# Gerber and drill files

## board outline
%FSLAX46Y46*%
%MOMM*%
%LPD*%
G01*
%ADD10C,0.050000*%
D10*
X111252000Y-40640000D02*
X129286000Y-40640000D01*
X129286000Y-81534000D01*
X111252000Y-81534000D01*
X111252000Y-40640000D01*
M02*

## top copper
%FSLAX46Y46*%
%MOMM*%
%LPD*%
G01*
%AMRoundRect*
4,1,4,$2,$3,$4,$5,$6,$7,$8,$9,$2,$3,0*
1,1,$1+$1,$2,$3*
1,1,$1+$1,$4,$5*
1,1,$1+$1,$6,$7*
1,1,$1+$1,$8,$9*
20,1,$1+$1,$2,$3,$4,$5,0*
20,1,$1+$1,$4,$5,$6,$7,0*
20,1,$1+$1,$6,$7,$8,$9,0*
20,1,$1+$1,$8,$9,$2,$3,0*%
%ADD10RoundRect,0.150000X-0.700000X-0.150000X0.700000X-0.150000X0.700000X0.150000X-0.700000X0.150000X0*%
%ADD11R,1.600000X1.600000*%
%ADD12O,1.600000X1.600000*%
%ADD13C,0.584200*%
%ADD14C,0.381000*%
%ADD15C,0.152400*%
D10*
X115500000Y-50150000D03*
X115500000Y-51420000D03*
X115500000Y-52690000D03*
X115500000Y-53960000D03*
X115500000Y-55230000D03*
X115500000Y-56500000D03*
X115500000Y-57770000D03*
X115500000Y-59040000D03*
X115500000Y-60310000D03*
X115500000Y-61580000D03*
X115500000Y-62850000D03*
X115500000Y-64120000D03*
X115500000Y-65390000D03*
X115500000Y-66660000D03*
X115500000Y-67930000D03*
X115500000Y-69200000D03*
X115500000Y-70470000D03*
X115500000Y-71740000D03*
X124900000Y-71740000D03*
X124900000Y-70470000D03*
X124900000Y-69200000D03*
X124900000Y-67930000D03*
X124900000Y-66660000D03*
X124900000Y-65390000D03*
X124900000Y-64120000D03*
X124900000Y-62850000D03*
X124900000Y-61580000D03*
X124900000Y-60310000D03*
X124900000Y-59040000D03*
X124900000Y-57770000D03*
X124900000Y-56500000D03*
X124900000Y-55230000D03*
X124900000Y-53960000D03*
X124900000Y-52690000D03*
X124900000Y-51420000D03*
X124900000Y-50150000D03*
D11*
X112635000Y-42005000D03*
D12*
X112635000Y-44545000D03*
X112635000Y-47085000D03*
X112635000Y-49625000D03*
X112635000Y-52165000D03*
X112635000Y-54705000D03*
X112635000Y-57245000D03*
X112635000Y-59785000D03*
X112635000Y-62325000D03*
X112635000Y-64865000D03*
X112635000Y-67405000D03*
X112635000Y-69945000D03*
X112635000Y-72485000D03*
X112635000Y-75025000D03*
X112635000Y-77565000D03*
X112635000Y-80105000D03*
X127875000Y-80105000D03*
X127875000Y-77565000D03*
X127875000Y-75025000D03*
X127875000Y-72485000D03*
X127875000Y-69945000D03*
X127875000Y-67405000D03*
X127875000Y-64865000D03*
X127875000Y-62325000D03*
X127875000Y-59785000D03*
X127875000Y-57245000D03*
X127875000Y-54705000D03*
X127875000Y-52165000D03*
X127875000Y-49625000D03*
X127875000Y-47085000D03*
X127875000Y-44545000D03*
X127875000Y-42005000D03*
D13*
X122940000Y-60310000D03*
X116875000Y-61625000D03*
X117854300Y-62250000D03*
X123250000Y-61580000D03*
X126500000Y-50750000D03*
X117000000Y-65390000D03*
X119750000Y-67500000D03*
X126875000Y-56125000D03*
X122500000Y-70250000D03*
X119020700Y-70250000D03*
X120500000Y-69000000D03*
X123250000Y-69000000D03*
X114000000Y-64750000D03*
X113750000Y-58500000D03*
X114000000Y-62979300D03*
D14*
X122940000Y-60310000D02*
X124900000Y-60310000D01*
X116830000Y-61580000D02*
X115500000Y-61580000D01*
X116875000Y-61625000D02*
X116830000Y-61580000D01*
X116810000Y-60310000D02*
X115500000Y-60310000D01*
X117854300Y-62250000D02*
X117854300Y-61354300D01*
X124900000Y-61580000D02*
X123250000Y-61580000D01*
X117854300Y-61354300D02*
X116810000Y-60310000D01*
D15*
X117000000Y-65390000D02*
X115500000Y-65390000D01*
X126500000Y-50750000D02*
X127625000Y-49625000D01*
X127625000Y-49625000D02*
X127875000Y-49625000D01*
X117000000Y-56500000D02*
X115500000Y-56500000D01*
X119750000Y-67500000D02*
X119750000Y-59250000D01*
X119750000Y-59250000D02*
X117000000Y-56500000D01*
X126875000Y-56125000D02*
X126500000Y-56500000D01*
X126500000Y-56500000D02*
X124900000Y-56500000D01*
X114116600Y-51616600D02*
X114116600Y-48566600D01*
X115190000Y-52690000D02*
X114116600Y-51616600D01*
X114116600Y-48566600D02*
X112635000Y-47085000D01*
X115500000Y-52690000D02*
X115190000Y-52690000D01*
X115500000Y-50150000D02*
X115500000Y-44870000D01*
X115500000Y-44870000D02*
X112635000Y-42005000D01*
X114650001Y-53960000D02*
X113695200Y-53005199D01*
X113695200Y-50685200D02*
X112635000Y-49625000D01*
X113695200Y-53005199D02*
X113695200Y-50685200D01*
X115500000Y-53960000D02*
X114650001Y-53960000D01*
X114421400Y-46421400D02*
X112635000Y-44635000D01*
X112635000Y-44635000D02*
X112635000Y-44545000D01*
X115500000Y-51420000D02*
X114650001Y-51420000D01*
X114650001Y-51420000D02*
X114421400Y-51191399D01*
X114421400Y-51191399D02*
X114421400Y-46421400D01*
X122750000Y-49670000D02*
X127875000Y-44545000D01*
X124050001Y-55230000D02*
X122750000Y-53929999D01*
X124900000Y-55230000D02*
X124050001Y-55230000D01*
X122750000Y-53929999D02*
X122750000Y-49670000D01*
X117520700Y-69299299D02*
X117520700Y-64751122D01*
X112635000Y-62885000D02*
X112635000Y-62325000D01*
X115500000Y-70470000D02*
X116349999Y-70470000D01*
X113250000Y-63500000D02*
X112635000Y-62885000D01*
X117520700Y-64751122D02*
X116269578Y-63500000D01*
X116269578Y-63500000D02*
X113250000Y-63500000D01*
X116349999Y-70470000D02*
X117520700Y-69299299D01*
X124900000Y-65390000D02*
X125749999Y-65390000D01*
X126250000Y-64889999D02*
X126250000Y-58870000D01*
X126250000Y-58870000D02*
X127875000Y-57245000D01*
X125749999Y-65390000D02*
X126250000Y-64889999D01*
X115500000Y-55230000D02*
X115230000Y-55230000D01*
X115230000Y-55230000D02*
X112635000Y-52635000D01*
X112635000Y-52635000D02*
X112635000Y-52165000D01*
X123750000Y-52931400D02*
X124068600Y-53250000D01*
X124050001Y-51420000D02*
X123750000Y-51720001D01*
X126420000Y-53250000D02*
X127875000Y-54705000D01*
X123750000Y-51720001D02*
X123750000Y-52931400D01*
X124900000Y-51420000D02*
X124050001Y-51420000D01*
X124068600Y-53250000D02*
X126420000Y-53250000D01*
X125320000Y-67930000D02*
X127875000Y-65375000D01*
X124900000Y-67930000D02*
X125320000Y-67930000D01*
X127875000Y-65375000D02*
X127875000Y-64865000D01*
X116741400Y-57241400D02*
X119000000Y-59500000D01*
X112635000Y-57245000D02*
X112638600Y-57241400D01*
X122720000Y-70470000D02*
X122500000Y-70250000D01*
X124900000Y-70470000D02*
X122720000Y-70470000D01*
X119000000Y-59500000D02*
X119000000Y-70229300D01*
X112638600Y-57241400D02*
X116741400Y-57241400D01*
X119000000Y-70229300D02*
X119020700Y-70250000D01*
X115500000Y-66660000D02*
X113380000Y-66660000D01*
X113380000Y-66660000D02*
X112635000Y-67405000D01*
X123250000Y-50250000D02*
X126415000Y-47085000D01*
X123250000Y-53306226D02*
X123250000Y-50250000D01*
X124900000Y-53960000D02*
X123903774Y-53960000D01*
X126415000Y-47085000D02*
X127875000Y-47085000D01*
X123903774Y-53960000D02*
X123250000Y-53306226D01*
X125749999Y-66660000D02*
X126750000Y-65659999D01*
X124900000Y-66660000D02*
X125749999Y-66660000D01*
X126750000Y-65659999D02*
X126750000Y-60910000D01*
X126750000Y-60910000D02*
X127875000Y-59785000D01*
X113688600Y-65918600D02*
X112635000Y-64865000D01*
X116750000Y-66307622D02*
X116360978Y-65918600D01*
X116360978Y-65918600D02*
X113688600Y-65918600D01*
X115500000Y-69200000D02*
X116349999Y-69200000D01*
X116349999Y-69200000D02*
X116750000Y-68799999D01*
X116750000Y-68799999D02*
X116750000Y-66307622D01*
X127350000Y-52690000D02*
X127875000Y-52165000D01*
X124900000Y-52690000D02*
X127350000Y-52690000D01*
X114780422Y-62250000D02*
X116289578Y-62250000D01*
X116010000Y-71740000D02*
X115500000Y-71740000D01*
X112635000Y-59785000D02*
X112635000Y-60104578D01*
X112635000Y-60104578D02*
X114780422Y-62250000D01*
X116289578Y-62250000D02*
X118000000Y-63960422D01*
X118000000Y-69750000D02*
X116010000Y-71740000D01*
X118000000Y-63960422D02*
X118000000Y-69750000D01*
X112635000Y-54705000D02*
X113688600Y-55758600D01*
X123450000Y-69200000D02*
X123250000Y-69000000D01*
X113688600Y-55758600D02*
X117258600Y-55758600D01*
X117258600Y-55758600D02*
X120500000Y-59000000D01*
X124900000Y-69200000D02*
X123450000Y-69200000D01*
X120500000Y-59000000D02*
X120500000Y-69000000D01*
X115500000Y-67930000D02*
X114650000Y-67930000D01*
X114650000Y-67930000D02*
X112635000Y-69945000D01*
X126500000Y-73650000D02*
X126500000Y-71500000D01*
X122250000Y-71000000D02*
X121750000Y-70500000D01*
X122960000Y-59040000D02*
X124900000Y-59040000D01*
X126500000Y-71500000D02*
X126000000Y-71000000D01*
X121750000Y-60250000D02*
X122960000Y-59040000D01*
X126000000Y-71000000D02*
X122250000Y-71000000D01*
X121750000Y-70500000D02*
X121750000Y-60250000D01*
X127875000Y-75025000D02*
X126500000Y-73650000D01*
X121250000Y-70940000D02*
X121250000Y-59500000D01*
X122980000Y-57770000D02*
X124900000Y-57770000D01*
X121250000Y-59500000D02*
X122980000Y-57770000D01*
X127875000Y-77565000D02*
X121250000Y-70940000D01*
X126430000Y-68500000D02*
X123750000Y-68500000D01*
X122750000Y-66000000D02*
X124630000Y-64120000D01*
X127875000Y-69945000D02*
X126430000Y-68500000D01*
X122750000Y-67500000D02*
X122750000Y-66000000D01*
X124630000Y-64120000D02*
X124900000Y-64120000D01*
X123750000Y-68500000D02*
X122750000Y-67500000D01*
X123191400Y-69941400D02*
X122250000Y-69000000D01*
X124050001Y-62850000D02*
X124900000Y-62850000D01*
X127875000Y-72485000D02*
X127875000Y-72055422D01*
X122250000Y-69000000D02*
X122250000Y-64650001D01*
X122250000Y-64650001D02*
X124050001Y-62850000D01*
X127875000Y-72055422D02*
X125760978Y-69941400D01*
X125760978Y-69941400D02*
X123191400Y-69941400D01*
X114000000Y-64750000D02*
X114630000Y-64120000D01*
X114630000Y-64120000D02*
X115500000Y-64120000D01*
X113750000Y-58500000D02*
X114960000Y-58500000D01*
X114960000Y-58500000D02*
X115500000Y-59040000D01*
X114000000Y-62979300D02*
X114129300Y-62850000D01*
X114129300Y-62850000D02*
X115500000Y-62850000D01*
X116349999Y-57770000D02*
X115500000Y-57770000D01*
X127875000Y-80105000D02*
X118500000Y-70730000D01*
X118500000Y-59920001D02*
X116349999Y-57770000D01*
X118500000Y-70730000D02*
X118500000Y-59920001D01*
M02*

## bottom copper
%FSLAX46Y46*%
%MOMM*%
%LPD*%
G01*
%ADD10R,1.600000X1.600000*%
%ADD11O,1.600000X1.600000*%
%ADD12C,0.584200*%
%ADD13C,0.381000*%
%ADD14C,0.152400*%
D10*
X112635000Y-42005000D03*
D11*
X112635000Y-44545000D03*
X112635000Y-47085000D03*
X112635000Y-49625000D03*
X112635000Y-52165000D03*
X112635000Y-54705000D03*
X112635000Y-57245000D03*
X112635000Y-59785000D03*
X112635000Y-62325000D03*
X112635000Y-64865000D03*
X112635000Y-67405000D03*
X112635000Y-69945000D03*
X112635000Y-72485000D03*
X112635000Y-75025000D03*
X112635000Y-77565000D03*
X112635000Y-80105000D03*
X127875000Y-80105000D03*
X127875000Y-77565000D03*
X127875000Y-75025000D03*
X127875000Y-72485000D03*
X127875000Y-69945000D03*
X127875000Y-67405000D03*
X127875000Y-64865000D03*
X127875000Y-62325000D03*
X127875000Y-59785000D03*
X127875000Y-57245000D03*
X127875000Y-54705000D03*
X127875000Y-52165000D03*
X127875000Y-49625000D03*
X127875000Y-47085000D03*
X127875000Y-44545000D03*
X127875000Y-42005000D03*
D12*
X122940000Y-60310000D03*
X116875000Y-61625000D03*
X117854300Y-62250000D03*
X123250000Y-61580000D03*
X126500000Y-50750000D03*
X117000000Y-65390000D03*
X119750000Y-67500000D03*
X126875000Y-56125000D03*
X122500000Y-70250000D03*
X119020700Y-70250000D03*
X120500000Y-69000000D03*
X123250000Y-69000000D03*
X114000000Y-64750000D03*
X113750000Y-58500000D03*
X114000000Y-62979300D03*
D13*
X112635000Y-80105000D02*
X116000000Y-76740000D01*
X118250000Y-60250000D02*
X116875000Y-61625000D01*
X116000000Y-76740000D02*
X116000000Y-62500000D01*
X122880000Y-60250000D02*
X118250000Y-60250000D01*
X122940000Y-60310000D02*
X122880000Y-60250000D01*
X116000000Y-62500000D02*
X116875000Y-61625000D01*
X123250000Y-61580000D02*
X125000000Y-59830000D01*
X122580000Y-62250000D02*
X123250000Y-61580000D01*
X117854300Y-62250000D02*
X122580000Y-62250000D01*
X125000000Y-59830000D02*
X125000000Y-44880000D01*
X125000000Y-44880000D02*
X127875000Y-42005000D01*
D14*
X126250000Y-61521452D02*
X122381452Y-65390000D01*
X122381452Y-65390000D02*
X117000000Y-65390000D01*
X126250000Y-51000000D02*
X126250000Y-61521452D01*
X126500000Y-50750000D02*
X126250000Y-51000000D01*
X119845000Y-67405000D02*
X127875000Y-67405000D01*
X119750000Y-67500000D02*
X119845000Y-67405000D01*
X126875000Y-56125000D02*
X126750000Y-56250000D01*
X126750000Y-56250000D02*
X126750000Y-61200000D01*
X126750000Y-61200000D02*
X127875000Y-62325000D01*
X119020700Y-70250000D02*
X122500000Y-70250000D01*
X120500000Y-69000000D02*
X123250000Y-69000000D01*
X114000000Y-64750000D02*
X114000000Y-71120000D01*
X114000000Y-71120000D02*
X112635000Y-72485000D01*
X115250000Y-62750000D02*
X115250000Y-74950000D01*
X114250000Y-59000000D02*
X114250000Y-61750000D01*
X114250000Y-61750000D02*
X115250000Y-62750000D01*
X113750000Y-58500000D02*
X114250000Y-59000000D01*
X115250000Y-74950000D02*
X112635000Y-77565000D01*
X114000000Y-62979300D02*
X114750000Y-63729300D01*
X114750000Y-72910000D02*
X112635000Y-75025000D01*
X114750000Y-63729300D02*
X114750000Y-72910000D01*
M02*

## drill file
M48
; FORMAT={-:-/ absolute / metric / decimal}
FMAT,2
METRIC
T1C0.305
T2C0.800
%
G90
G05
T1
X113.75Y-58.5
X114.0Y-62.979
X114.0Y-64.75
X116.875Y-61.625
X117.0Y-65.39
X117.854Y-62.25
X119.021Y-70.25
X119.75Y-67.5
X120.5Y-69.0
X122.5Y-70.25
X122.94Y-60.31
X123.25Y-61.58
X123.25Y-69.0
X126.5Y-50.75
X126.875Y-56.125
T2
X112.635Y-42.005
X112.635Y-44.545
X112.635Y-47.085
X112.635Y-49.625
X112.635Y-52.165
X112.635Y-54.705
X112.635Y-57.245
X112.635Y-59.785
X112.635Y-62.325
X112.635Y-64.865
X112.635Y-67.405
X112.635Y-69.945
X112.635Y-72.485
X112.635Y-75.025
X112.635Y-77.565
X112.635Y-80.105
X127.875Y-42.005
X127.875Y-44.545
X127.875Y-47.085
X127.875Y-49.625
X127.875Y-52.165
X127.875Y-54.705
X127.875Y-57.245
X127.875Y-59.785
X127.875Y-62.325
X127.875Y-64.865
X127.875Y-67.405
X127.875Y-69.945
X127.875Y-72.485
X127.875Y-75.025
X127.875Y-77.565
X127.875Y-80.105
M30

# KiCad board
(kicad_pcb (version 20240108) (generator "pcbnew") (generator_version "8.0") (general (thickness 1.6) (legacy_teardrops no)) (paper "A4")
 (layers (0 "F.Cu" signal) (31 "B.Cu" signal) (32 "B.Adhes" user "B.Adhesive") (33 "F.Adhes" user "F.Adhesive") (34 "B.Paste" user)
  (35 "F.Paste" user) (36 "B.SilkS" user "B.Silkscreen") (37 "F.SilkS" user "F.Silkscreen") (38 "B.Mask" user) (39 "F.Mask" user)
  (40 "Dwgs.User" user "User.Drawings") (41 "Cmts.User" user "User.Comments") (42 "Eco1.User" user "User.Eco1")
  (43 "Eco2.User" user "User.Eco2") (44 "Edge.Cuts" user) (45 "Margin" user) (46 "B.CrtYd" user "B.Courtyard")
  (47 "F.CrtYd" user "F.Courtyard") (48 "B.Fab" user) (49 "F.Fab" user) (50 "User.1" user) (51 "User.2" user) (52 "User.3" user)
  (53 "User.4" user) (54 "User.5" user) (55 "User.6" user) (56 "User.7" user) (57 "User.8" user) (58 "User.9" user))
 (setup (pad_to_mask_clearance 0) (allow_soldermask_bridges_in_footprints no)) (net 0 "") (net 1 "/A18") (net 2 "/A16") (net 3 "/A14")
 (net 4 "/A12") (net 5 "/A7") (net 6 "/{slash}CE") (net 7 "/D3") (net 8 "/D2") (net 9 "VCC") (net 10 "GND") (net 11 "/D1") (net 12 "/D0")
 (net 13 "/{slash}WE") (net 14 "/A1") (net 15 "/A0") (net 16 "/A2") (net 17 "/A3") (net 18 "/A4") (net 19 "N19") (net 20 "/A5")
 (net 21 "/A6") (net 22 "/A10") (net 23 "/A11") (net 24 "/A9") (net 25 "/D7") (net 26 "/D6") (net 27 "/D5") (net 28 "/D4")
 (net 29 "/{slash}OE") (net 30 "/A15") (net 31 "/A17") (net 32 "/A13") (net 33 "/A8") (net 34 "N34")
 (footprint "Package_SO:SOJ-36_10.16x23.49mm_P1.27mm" (layer "F.Cu") (at 120.2 60.945)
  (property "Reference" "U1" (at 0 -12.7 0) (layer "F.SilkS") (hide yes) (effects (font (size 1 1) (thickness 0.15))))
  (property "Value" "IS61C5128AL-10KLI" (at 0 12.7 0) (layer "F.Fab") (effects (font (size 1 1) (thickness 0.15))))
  (pad "1" smd roundrect (at -4.7 -10.795) (size 1.7 0.6) (layers "F.Cu" "F.Paste" "F.Mask") (roundrect_rratio 0.25) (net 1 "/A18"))
  (pad "2" smd roundrect (at -4.7 -9.525) (size 1.7 0.6) (layers "F.Cu" "F.Paste" "F.Mask") (roundrect_rratio 0.25) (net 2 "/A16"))
  (pad "3" smd roundrect (at -4.7 -8.255) (size 1.7 0.6) (layers "F.Cu" "F.Paste" "F.Mask") (roundrect_rratio 0.25) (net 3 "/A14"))
  (pad "4" smd roundrect (at -4.7 -6.985) (size 1.7 0.6) (layers "F.Cu" "F.Paste" "F.Mask") (roundrect_rratio 0.25) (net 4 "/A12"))
  (pad "5" smd roundrect (at -4.7 -5.715) (size 1.7 0.6) (layers "F.Cu" "F.Paste" "F.Mask") (roundrect_rratio 0.25) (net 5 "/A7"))
  (pad "6" smd roundrect (at -4.7 -4.445) (size 1.7 0.6) (layers "F.Cu" "F.Paste" "F.Mask") (roundrect_rratio 0.25) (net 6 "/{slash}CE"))
  (pad "7" smd roundrect (at -4.7 -3.175) (size 1.7 0.6) (layers "F.Cu" "F.Paste" "F.Mask") (roundrect_rratio 0.25) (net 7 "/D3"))
  (pad "8" smd roundrect (at -4.7 -1.905) (size 1.7 0.6) (layers "F.Cu" "F.Paste" "F.Mask") (roundrect_rratio 0.25) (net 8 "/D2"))
  (pad "9" smd roundrect (at -4.7 -0.635) (size 1.7 0.6) (layers "F.Cu" "F.Paste" "F.Mask") (roundrect_rratio 0.25) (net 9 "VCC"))
  (pad "10" smd roundrect (at -4.7 0.635) (size 1.7 0.6) (layers "F.Cu" "F.Paste" "F.Mask") (roundrect_rratio 0.25) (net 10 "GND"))
  (pad "11" smd roundrect (at -4.7 1.905) (size 1.7 0.6) (layers "F.Cu" "F.Paste" "F.Mask") (roundrect_rratio 0.25) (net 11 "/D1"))
  (pad "12" smd roundrect (at -4.7 3.175) (size 1.7 0.6) (layers "F.Cu" "F.Paste" "F.Mask") (roundrect_rratio 0.25) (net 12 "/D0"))
  (pad "13" smd roundrect (at -4.7 4.445) (size 1.7 0.6) (layers "F.Cu" "F.Paste" "F.Mask") (roundrect_rratio 0.25) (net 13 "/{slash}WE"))
  (pad "14" smd roundrect (at -4.7 5.715) (size 1.7 0.6) (layers "F.Cu" "F.Paste" "F.Mask") (roundrect_rratio 0.25) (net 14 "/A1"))
  (pad "15" smd roundrect (at -4.7 6.985) (size 1.7 0.6) (layers "F.Cu" "F.Paste" "F.Mask") (roundrect_rratio 0.25) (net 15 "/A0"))
  (pad "16" smd roundrect (at -4.7 8.255) (size 1.7 0.6) (layers "F.Cu" "F.Paste" "F.Mask") (roundrect_rratio 0.25) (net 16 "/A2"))
  (pad "17" smd roundrect (at -4.7 9.525) (size 1.7 0.6) (layers "F.Cu" "F.Paste" "F.Mask") (roundrect_rratio 0.25) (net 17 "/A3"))
  (pad "18" smd roundrect (at -4.7 10.795) (size 1.7 0.6) (layers "F.Cu" "F.Paste" "F.Mask") (roundrect_rratio 0.25) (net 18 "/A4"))
  (pad "19" smd roundrect (at 4.7 10.795) (size 1.7 0.6) (layers "F.Cu" "F.Paste" "F.Mask") (roundrect_rratio 0.25) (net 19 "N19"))
  (pad "20" smd roundrect (at 4.7 9.525) (size 1.7 0.6) (layers "F.Cu" "F.Paste" "F.Mask") (roundrect_rratio 0.25) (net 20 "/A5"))
  (pad "21" smd roundrect (at 4.7 8.255) (size 1.7 0.6) (layers "F.Cu" "F.Paste" "F.Mask") (roundrect_rratio 0.25) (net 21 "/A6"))
  (pad "22" smd roundrect (at 4.7 6.985) (size 1.7 0.6) (layers "F.Cu" "F.Paste" "F.Mask") (roundrect_rratio 0.25) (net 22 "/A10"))
  (pad "23" smd roundrect (at 4.7 5.715) (size 1.7 0.6) (layers "F.Cu" "F.Paste" "F.Mask") (roundrect_rratio 0.25) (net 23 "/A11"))
  (pad "24" smd roundrect (at 4.7 4.445) (size 1.7 0.6) (layers "F.Cu" "F.Paste" "F.Mask") (roundrect_rratio 0.25) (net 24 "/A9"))
  (pad "25" smd roundrect (at 4.7 3.175) (size 1.7 0.6) (layers "F.Cu" "F.Paste" "F.Mask") (roundrect_rratio 0.25) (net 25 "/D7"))
  (pad "26" smd roundrect (at 4.7 1.905) (size 1.7 0.6) (layers "F.Cu" "F.Paste" "F.Mask") (roundrect_rratio 0.25) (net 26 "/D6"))
  (pad "27" smd roundrect (at 4.7 0.635) (size 1.7 0.6) (layers "F.Cu" "F.Paste" "F.Mask") (roundrect_rratio 0.25) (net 9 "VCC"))
  (pad "28" smd roundrect (at 4.7 -0.635) (size 1.7 0.6) (layers "F.Cu" "F.Paste" "F.Mask") (roundrect_rratio 0.25) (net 10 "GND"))
  (pad "29" smd roundrect (at 4.7 -1.905) (size 1.7 0.6) (layers "F.Cu" "F.Paste" "F.Mask") (roundrect_rratio 0.25) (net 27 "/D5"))
  (pad "30" smd roundrect (at 4.7 -3.175) (size 1.7 0.6) (layers "F.Cu" "F.Paste" "F.Mask") (roundrect_rratio 0.25) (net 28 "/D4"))
  (pad "31" smd roundrect (at 4.7 -4.445) (size 1.7 0.6) (layers "F.Cu" "F.Paste" "F.Mask") (roundrect_rratio 0.25) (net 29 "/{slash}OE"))
  (pad "32" smd roundrect (at 4.7 -5.715) (size 1.7 0.6) (layers "F.Cu" "F.Paste" "F.Mask") (roundrect_rratio 0.25) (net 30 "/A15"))
  (pad "33" smd roundrect (at 4.7 -6.985) (size 1.7 0.6) (layers "F.Cu" "F.Paste" "F.Mask") (roundrect_rratio 0.25) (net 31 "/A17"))
  (pad "34" smd roundrect (at 4.7 -8.255) (size 1.7 0.6) (layers "F.Cu" "F.Paste" "F.Mask") (roundrect_rratio 0.25) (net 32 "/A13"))
  (pad "35" smd roundrect (at 4.7 -9.525) (size 1.7 0.6) (layers "F.Cu" "F.Paste" "F.Mask") (roundrect_rratio 0.25) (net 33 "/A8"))
  (pad "36" smd roundrect (at 4.7 -10.795) (size 1.7 0.6) (layers "F.Cu" "F.Paste" "F.Mask") (roundrect_rratio 0.25) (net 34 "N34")))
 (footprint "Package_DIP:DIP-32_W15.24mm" (layer "F.Cu") (at 112.635 42.005)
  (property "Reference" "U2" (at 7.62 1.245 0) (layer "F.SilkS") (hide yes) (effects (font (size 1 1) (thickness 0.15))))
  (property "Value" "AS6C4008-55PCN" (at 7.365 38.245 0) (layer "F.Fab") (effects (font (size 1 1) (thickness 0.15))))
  (pad "1" thru_hole rect (at 0 0) (size 1.6 1.6) (drill 0.8) (layers "*.Cu" "*.Mask") (remove_unused_layers no) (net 1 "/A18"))
  (pad "2" thru_hole oval (at 0 2.54) (size 1.6 1.6) (drill 0.8) (layers "*.Cu" "*.Mask") (remove_unused_layers no) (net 2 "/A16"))
  (pad "3" thru_hole oval (at 0 5.08) (size 1.6 1.6) (drill 0.8) (layers "*.Cu" "*.Mask") (remove_unused_layers no) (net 3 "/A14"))
  (pad "4" thru_hole oval (at 0 7.62) (size 1.6 1.6) (drill 0.8) (layers "*.Cu" "*.Mask") (remove_unused_layers no) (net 4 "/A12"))
  (pad "5" thru_hole oval (at 0 10.16) (size 1.6 1.6) (drill 0.8) (layers "*.Cu" "*.Mask") (remove_unused_layers no) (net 5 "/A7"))
  (pad "6" thru_hole oval (at 0 12.7) (size 1.6 1.6) (drill 0.8) (layers "*.Cu" "*.Mask") (remove_unused_layers no) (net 21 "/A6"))
  (pad "7" thru_hole oval (at 0 15.24) (size 1.6 1.6) (drill 0.8) (layers "*.Cu" "*.Mask") (remove_unused_layers no) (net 20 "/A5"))
  (pad "8" thru_hole oval (at 0 17.78) (size 1.6 1.6) (drill 0.8) (layers "*.Cu" "*.Mask") (remove_unused_layers no) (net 18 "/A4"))
  (pad "9" thru_hole oval (at 0 20.32) (size 1.6 1.6) (drill 0.8) (layers "*.Cu" "*.Mask") (remove_unused_layers no) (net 17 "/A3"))
  (pad "10" thru_hole oval (at 0 22.86) (size 1.6 1.6) (drill 0.8) (layers "*.Cu" "*.Mask") (remove_unused_layers no) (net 16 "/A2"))
  (pad "11" thru_hole oval (at 0 25.4) (size 1.6 1.6) (drill 0.8) (layers "*.Cu" "*.Mask") (remove_unused_layers no) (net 14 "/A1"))
  (pad "12" thru_hole oval (at 0 27.94) (size 1.6 1.6) (drill 0.8) (layers "*.Cu" "*.Mask") (remove_unused_layers no) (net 15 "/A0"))
  (pad "13" thru_hole oval (at 0 30.48) (size 1.6 1.6) (drill 0.8) (layers "*.Cu" "*.Mask") (remove_unused_layers no) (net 12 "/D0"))
  (pad "14" thru_hole oval (at 0 33.02) (size 1.6 1.6) (drill 0.8) (layers "*.Cu" "*.Mask") (remove_unused_layers no) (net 11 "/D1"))
  (pad "15" thru_hole oval (at 0 35.56) (size 1.6 1.6) (drill 0.8) (layers "*.Cu" "*.Mask") (remove_unused_layers no) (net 8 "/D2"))
  (pad "16" thru_hole oval (at 0 38.1) (size 1.6 1.6) (drill 0.8) (layers "*.Cu" "*.Mask") (remove_unused_layers no) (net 10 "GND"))
  (pad "17" thru_hole oval (at 15.24 38.1) (size 1.6 1.6) (drill 0.8) (layers "*.Cu" "*.Mask") (remove_unused_layers no) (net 7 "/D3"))
  (pad "18" thru_hole oval (at 15.24 35.56) (size 1.6 1.6) (drill 0.8) (layers "*.Cu" "*.Mask") (remove_unused_layers no) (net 28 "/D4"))
  (pad "19" thru_hole oval (at 15.24 33.02) (size 1.6 1.6) (drill 0.8) (layers "*.Cu" "*.Mask") (remove_unused_layers no) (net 27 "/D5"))
  (pad "20" thru_hole oval (at 15.24 30.48) (size 1.6 1.6) (drill 0.8) (layers "*.Cu" "*.Mask") (remove_unused_layers no) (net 26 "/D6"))
  (pad "21" thru_hole oval (at 15.24 27.94) (size 1.6 1.6) (drill 0.8) (layers "*.Cu" "*.Mask") (remove_unused_layers no) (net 25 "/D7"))
  (pad "22" thru_hole oval (at 15.24 25.4) (size 1.6 1.6) (drill 0.8) (layers "*.Cu" "*.Mask") (remove_unused_layers no)
   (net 6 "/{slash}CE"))
  (pad "23" thru_hole oval (at 15.24 22.86) (size 1.6 1.6) (drill 0.8) (layers "*.Cu" "*.Mask") (remove_unused_layers no) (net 22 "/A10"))
  (pad "24" thru_hole oval (at 15.24 20.32) (size 1.6 1.6) (drill 0.8) (layers "*.Cu" "*.Mask") (remove_unused_layers no)
   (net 29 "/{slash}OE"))
  (pad "25" thru_hole oval (at 15.24 17.78) (size 1.6 1.6) (drill 0.8) (layers "*.Cu" "*.Mask") (remove_unused_layers no) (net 23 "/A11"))
  (pad "26" thru_hole oval (at 15.24 15.24) (size 1.6 1.6) (drill 0.8) (layers "*.Cu" "*.Mask") (remove_unused_layers no) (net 24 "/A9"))
  (pad "27" thru_hole oval (at 15.24 12.7) (size 1.6 1.6) (drill 0.8) (layers "*.Cu" "*.Mask") (remove_unused_layers no) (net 33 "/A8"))
  (pad "28" thru_hole oval (at 15.24 10.16) (size 1.6 1.6) (drill 0.8) (layers "*.Cu" "*.Mask") (remove_unused_layers no) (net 32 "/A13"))
  (pad "29" thru_hole oval (at 15.24 7.62) (size 1.6 1.6) (drill 0.8) (layers "*.Cu" "*.Mask") (remove_unused_layers no)
   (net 13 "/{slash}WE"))
  (pad "30" thru_hole oval (at 15.24 5.08) (size 1.6 1.6) (drill 0.8) (layers "*.Cu" "*.Mask") (remove_unused_layers no) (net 31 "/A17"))
  (pad "31" thru_hole oval (at 15.24 2.54) (size 1.6 1.6) (drill 0.8) (layers "*.Cu" "*.Mask") (remove_unused_layers no) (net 30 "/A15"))
  (pad "32" thru_hole oval (at 15.24 0) (size 1.6 1.6) (drill 0.8) (layers "*.Cu" "*.Mask") (remove_unused_layers no) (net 9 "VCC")))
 (gr_rect (start 111.252 40.64) (end 129.286 81.534) (stroke (width 0.05) (type default)) (fill none) (layer "Edge.Cuts"))
 (segment (start 122.94 60.31) (end 124.9 60.31) (width 0.381) (layer "F.Cu") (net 10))
 (segment (start 116.83 61.58) (end 115.5 61.58) (width 0.381) (layer "F.Cu") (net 10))
 (segment (start 116.875 61.625) (end 116.83 61.58) (width 0.381) (layer "F.Cu") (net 10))
 (via (at 122.94 60.31) (size 0.5842) (drill 0.3048) (layers "F.Cu" "B.Cu") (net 10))
 (via (at 116.875 61.625) (size 0.5842) (drill 0.3048) (layers "F.Cu" "B.Cu") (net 10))
 (segment (start 112.635 80.105) (end 116 76.74) (width 0.381) (layer "B.Cu") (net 10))
 (segment (start 118.25 60.25) (end 116.875 61.625) (width 0.381) (layer "B.Cu") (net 10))
 (segment (start 116 76.74) (end 116 62.5) (width 0.381) (layer "B.Cu") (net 10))
 (segment (start 122.88 60.25) (end 118.25 60.25) (width 0.381) (layer "B.Cu") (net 10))
 (segment (start 122.94 60.31) (end 122.88 60.25) (width 0.381) (layer "B.Cu") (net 10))
 (segment (start 116 62.5) (end 116.875 61.625) (width 0.381) (layer "B.Cu") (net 10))
 (segment (start 116.81 60.31) (end 115.5 60.31) (width 0.381) (layer "F.Cu") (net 9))
 (segment (start 117.8543 62.25) (end 117.8543 61.3543) (width 0.381) (layer "F.Cu") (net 9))
 (segment (start 124.9 61.58) (end 123.25 61.58) (width 0.381) (layer "F.Cu") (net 9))
 (segment (start 117.8543 61.3543) (end 116.81 60.31) (width 0.381) (layer "F.Cu") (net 9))
 (via (at 117.8543 62.25) (size 0.5842) (drill 0.3048) (layers "F.Cu" "B.Cu") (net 9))
 (via (at 123.25 61.58) (size 0.5842) (drill 0.3048) (layers "F.Cu" "B.Cu") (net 9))
 (segment (start 123.25 61.58) (end 125 59.83) (width 0.381) (layer "B.Cu") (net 9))
 (segment (start 122.58 62.25) (end 123.25 61.58) (width 0.381) (layer "B.Cu") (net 9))
 (segment (start 117.8543 62.25) (end 122.58 62.25) (width 0.381) (layer "B.Cu") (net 9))
 (segment (start 125 59.83) (end 125 44.88) (width 0.381) (layer "B.Cu") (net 9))
 (segment (start 125 44.88) (end 127.875 42.005) (width 0.381) (layer "B.Cu") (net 9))
 (segment (start 117 65.39) (end 115.5 65.39) (width 0.1524) (layer "F.Cu") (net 13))
 (segment (start 126.5 50.75) (end 127.625 49.625) (width 0.1524) (layer "F.Cu") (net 13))
 (segment (start 127.625 49.625) (end 127.875 49.625) (width 0.1524) (layer "F.Cu") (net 13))
 (via (at 126.5 50.75) (size 0.5842) (drill 0.3048) (layers "F.Cu" "B.Cu") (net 13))
 (via (at 117 65.39) (size 0.5842) (drill 0.3048) (layers "F.Cu" "B.Cu") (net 13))
 (segment (start 126.25 61.521452) (end 122.381452 65.39) (width 0.1524) (layer "B.Cu") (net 13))
 (segment (start 122.381452 65.39) (end 117 65.39) (width 0.1524) (layer "B.Cu") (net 13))
 (segment (start 126.25 51) (end 126.25 61.521452) (width 0.1524) (layer "B.Cu") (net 13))
 (segment (start 126.5 50.75) (end 126.25 51) (width 0.1524) (layer "B.Cu") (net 13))
 (segment (start 117 56.5) (end 115.5 56.5) (width 0.1524) (layer "F.Cu") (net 6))
 (segment (start 119.75 67.5) (end 119.75 59.25) (width 0.1524) (layer "F.Cu") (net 6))
 (segment (start 119.75 59.25) (end 117 56.5) (width 0.1524) (layer "F.Cu") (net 6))
 (via (at 119.75 67.5) (size 0.5842) (drill 0.3048) (layers "F.Cu" "B.Cu") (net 6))
 (segment (start 119.845 67.405) (end 127.875 67.405) (width 0.1524) (layer "B.Cu") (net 6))
 (segment (start 119.75 67.5) (end 119.845 67.405) (width 0.1524) (layer "B.Cu") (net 6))
 (segment (start 126.875 56.125) (end 126.5 56.5) (width 0.1524) (layer "F.Cu") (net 29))
 (segment (start 126.5 56.5) (end 124.9 56.5) (width 0.1524) (layer "F.Cu") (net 29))
 (via (at 126.875 56.125) (size 0.5842) (drill 0.3048) (layers "F.Cu" "B.Cu") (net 29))
 (segment (start 126.875 56.125) (end 126.75 56.25) (width 0.1524) (layer "B.Cu") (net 29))
 (segment (start 126.75 56.25) (end 126.75 61.2) (width 0.1524) (layer "B.Cu") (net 29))
 (segment (start 126.75 61.2) (end 127.875 62.325) (width 0.1524) (layer "B.Cu") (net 29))
 (segment (start 114.1166 51.6166) (end 114.1166 48.5666) (width 0.1524) (layer "F.Cu") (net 3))
 (segment (start 115.19 52.69) (end 114.1166 51.6166) (width 0.1524) (layer "F.Cu") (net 3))
 (segment (start 114.1166 48.5666) (end 112.635 47.085) (width 0.1524) (layer "F.Cu") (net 3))
 (segment (start 115.5 52.69) (end 115.19 52.69) (width 0.1524) (layer "F.Cu") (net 3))
 (segment (start 115.5 50.15) (end 115.5 44.87) (width 0.1524) (layer "F.Cu") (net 1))
 (segment (start 115.5 44.87) (end 112.635 42.005) (width 0.1524) (layer "F.Cu") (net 1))
 (segment (start 114.650001 53.96) (end 113.6952 53.005199) (width 0.1524) (layer "F.Cu") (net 4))
 (segment (start 113.6952 50.6852) (end 112.635 49.625) (width 0.1524) (layer "F.Cu") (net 4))
 (segment (start 113.6952 53.005199) (end 113.6952 50.6852) (width 0.1524) (layer "F.Cu") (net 4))
 (segment (start 115.5 53.96) (end 114.650001 53.96) (width 0.1524) (layer "F.Cu") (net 4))
 (segment (start 114.4214 46.4214) (end 112.635 44.635) (width 0.1524) (layer "F.Cu") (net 2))
 (segment (start 112.635 44.635) (end 112.635 44.545) (width 0.1524) (layer "F.Cu") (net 2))
 (segment (start 115.5 51.42) (end 114.650001 51.42) (width 0.1524) (layer "F.Cu") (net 2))
 (segment (start 114.650001 51.42) (end 114.4214 51.191399) (width 0.1524) (layer "F.Cu") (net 2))
 (segment (start 114.4214 51.191399) (end 114.4214 46.4214) (width 0.1524) (layer "F.Cu") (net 2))
 (segment (start 122.75 49.67) (end 127.875 44.545) (width 0.1524) (layer "F.Cu") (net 30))
 (segment (start 124.050001 55.23) (end 122.75 53.929999) (width 0.1524) (layer "F.Cu") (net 30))
 (segment (start 124.9 55.23) (end 124.050001 55.23) (width 0.1524) (layer "F.Cu") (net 30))
 (segment (start 122.75 53.929999) (end 122.75 49.67) (width 0.1524) (layer "F.Cu") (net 30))
 (segment (start 117.5207 69.299299) (end 117.5207 64.751122) (width 0.1524) (layer "F.Cu") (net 17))
 (segment (start 112.635 62.885) (end 112.635 62.325) (width 0.1524) (layer "F.Cu") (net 17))
 (segment (start 115.5 70.47) (end 116.349999 70.47) (width 0.1524) (layer "F.Cu") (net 17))
 (segment (start 113.25 63.5) (end 112.635 62.885) (width 0.1524) (layer "F.Cu") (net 17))
 (segment (start 117.5207 64.751122) (end 116.269578 63.5) (width 0.1524) (layer "F.Cu") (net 17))
 (segment (start 116.269578 63.5) (end 113.25 63.5) (width 0.1524) (layer "F.Cu") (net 17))
 (segment (start 116.349999 70.47) (end 117.5207 69.299299) (width 0.1524) (layer "F.Cu") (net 17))
 (segment (start 124.9 65.39) (end 125.749999 65.39) (width 0.1524) (layer "F.Cu") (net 24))
 (segment (start 126.25 64.889999) (end 126.25 58.87) (width 0.1524) (layer "F.Cu") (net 24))
 (segment (start 126.25 58.87) (end 127.875 57.245) (width 0.1524) (layer "F.Cu") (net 24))
 (segment (start 125.749999 65.39) (end 126.25 64.889999) (width 0.1524) (layer "F.Cu") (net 24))
 (segment (start 115.5 55.23) (end 115.23 55.23) (width 0.1524) (layer "F.Cu") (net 5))
 (segment (start 115.23 55.23) (end 112.635 52.635) (width 0.1524) (layer "F.Cu") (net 5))
 (segment (start 112.635 52.635) (end 112.635 52.165) (width 0.1524) (layer "F.Cu") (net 5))
 (segment (start 123.75 52.9314) (end 124.0686 53.25) (width 0.1524) (layer "F.Cu") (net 33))
 (segment (start 124.050001 51.42) (end 123.75 51.720001) (width 0.1524) (layer "F.Cu") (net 33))
 (segment (start 126.42 53.25) (end 127.875 54.705) (width 0.1524) (layer "F.Cu") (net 33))
 (segment (start 123.75 51.720001) (end 123.75 52.9314) (width 0.1524) (layer "F.Cu") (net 33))
 (segment (start 124.9 51.42) (end 124.050001 51.42) (width 0.1524) (layer "F.Cu") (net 33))
 (segment (start 124.0686 53.25) (end 126.42 53.25) (width 0.1524) (layer "F.Cu") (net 33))
 (segment (start 125.32 67.93) (end 127.875 65.375) (width 0.1524) (layer "F.Cu") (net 22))
 (segment (start 124.9 67.93) (end 125.32 67.93) (width 0.1524) (layer "F.Cu") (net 22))
 (segment (start 127.875 65.375) (end 127.875 64.865) (width 0.1524) (layer "F.Cu") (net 22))
 (segment (start 116.7414 57.2414) (end 119 59.5) (width 0.1524) (layer "F.Cu") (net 20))
 (segment (start 112.635 57.245) (end 112.6386 57.2414) (width 0.1524) (layer "F.Cu") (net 20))
 (segment (start 122.72 70.47) (end 122.5 70.25) (width 0.1524) (layer "F.Cu") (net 20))
 (segment (start 124.9 70.47) (end 122.72 70.47) (width 0.1524) (layer "F.Cu") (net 20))
 (segment (start 119 59.5) (end 119 70.2293) (width 0.1524) (layer "F.Cu") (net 20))
 (segment (start 112.6386 57.2414) (end 116.7414 57.2414) (width 0.1524) (layer "F.Cu") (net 20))
 (segment (start 119 70.2293) (end 119.0207 70.25) (width 0.1524) (layer "F.Cu") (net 20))
 (via (at 122.5 70.25) (size 0.5842) (drill 0.3048) (layers "F.Cu" "B.Cu") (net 20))
 (via (at 119.0207 70.25) (size 0.5842) (drill 0.3048) (layers "F.Cu" "B.Cu") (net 20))
 (segment (start 119.0207 70.25) (end 122.5 70.25) (width 0.1524) (layer "B.Cu") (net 20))
 (segment (start 115.5 66.66) (end 113.38 66.66) (width 0.1524) (layer "F.Cu") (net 14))
 (segment (start 113.38 66.66) (end 112.635 67.405) (width 0.1524) (layer "F.Cu") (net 14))
 (segment (start 123.25 50.25) (end 126.415 47.085) (width 0.1524) (layer "F.Cu") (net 31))
 (segment (start 123.25 53.306226) (end 123.25 50.25) (width 0.1524) (layer "F.Cu") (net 31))
 (segment (start 124.9 53.96) (end 123.903774 53.96) (width 0.1524) (layer "F.Cu") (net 31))
 (segment (start 126.415 47.085) (end 127.875 47.085) (width 0.1524) (layer "F.Cu") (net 31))
 (segment (start 123.903774 53.96) (end 123.25 53.306226) (width 0.1524) (layer "F.Cu") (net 31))
 (segment (start 125.749999 66.66) (end 126.75 65.659999) (width 0.1524) (layer "F.Cu") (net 23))
 (segment (start 124.9 66.66) (end 125.749999 66.66) (width 0.1524) (layer "F.Cu") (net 23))
 (segment (start 126.75 65.659999) (end 126.75 60.91) (width 0.1524) (layer "F.Cu") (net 23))
 (segment (start 126.75 60.91) (end 127.875 59.785) (width 0.1524) (layer "F.Cu") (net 23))
 (segment (start 113.6886 65.9186) (end 112.635 64.865) (width 0.1524) (layer "F.Cu") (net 16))
 (segment (start 116.75 66.307622) (end 116.360978 65.9186) (width 0.1524) (layer "F.Cu") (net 16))
 (segment (start 116.360978 65.9186) (end 113.6886 65.9186) (width 0.1524) (layer "F.Cu") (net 16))
 (segment (start 115.5 69.2) (end 116.349999 69.2) (width 0.1524) (layer "F.Cu") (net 16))
 (segment (start 116.349999 69.2) (end 116.75 68.799999) (width 0.1524) (layer "F.Cu") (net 16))
 (segment (start 116.75 68.799999) (end 116.75 66.307622) (width 0.1524) (layer "F.Cu") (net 16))
 (segment (start 127.35 52.69) (end 127.875 52.165) (width 0.1524) (layer "F.Cu") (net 32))
 (segment (start 124.9 52.69) (end 127.35 52.69) (width 0.1524) (layer "F.Cu") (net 32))
 (segment (start 114.780422 62.25) (end 116.289578 62.25) (width 0.1524) (layer "F.Cu") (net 18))
 (segment (start 116.01 71.74) (end 115.5 71.74) (width 0.1524) (layer "F.Cu") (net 18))
 (segment (start 112.635 59.785) (end 112.635 60.104578) (width 0.1524) (layer "F.Cu") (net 18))
 (segment (start 112.635 60.104578) (end 114.780422 62.25) (width 0.1524) (layer "F.Cu") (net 18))
 (segment (start 116.289578 62.25) (end 118 63.960422) (width 0.1524) (layer "F.Cu") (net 18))
 (segment (start 118 69.75) (end 116.01 71.74) (width 0.1524) (layer "F.Cu") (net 18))
 (segment (start 118 63.960422) (end 118 69.75) (width 0.1524) (layer "F.Cu") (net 18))
 (segment (start 112.635 54.705) (end 113.6886 55.7586) (width 0.1524) (layer "F.Cu") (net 21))
 (segment (start 123.45 69.2) (end 123.25 69) (width 0.1524) (layer "F.Cu") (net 21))
 (segment (start 113.6886 55.7586) (end 117.2586 55.7586) (width 0.1524) (layer "F.Cu") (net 21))
 (segment (start 117.2586 55.7586) (end 120.5 59) (width 0.1524) (layer "F.Cu") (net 21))
 (segment (start 124.9 69.2) (end 123.45 69.2) (width 0.1524) (layer "F.Cu") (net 21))
 (segment (start 120.5 59) (end 120.5 69) (width 0.1524) (layer "F.Cu") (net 21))
 (via (at 120.5 69) (size 0.5842) (drill 0.3048) (layers "F.Cu" "B.Cu") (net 21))
 (via (at 123.25 69) (size 0.5842) (drill 0.3048) (layers "F.Cu" "B.Cu") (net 21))
 (segment (start 120.5 69) (end 123.25 69) (width 0.1524) (layer "B.Cu") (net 21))
 (segment (start 115.5 67.93) (end 114.65 67.93) (width 0.1524) (layer "F.Cu") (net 15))
 (segment (start 114.65 67.93) (end 112.635 69.945) (width 0.1524) (layer "F.Cu") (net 15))
 (segment (start 126.5 73.65) (end 126.5 71.5) (width 0.1524) (layer "F.Cu") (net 27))
 (segment (start 122.25 71) (end 121.75 70.5) (width 0.1524) (layer "F.Cu") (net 27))
 (segment (start 122.96 59.04) (end 124.9 59.04) (width 0.1524) (layer "F.Cu") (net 27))
 (segment (start 126.5 71.5) (end 126 71) (width 0.1524) (layer "F.Cu") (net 27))
 (segment (start 121.75 60.25) (end 122.96 59.04) (width 0.1524) (layer "F.Cu") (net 27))
 (segment (start 126 71) (end 122.25 71) (width 0.1524) (layer "F.Cu") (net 27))
 (segment (start 121.75 70.5) (end 121.75 60.25) (width 0.1524) (layer "F.Cu") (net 27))
 (segment (start 127.875 75.025) (end 126.5 73.65) (width 0.1524) (layer "F.Cu") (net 27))
 (segment (start 121.25 70.94) (end 121.25 59.5) (width 0.1524) (layer "F.Cu") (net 28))
 (segment (start 122.98 57.77) (end 124.9 57.77) (width 0.1524) (layer "F.Cu") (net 28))
 (segment (start 121.25 59.5) (end 122.98 57.77) (width 0.1524) (layer "F.Cu") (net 28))
 (segment (start 127.875 77.565) (end 121.25 70.94) (width 0.1524) (layer "F.Cu") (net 28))
 (segment (start 126.43 68.5) (end 123.75 68.5) (width 0.1524) (layer "F.Cu") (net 25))
 (segment (start 122.75 66) (end 124.63 64.12) (width 0.1524) (layer "F.Cu") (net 25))
 (segment (start 127.875 69.945) (end 126.43 68.5) (width 0.1524) (layer "F.Cu") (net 25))
 (segment (start 122.75 67.5) (end 122.75 66) (width 0.1524) (layer "F.Cu") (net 25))
 (segment (start 124.63 64.12) (end 124.9 64.12) (width 0.1524) (layer "F.Cu") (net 25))
 (segment (start 123.75 68.5) (end 122.75 67.5) (width 0.1524) (layer "F.Cu") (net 25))
 (segment (start 123.1914 69.9414) (end 122.25 69) (width 0.1524) (layer "F.Cu") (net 26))
 (segment (start 124.050001 62.85) (end 124.9 62.85) (width 0.1524) (layer "F.Cu") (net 26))
 (segment (start 127.875 72.485) (end 127.875 72.055422) (width 0.1524) (layer "F.Cu") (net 26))
 (segment (start 122.25 69) (end 122.25 64.650001) (width 0.1524) (layer "F.Cu") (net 26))
 (segment (start 122.25 64.650001) (end 124.050001 62.85) (width 0.1524) (layer "F.Cu") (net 26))
 (segment (start 127.875 72.055422) (end 125.760978 69.9414) (width 0.1524) (layer "F.Cu") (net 26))
 (segment (start 125.760978 69.9414) (end 123.1914 69.9414) (width 0.1524) (layer "F.Cu") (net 26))
 (segment (start 114 64.75) (end 114.63 64.12) (width 0.1524) (layer "F.Cu") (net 12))
 (segment (start 114.63 64.12) (end 115.5 64.12) (width 0.1524) (layer "F.Cu") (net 12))
 (via (at 114 64.75) (size 0.5842) (drill 0.3048) (layers "F.Cu" "B.Cu") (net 12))
 (segment (start 114 64.75) (end 114 71.12) (width 0.1524) (layer "B.Cu") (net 12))
 (segment (start 114 71.12) (end 112.635 72.485) (width 0.1524) (layer "B.Cu") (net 12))
 (segment (start 113.75 58.5) (end 114.96 58.5) (width 0.1524) (layer "F.Cu") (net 8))
 (segment (start 114.96 58.5) (end 115.5 59.04) (width 0.1524) (layer "F.Cu") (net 8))
 (via (at 113.75 58.5) (size 0.5842) (drill 0.3048) (layers "F.Cu" "B.Cu") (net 8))
 (segment (start 115.25 62.75) (end 115.25 74.95) (width 0.1524) (layer "B.Cu") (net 8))
 (segment (start 114.25 59) (end 114.25 61.75) (width 0.1524) (layer "B.Cu") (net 8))
 (segment (start 114.25 61.75) (end 115.25 62.75) (width 0.1524) (layer "B.Cu") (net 8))
 (segment (start 113.75 58.5) (end 114.25 59) (width 0.1524) (layer "B.Cu") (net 8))
 (segment (start 115.25 74.95) (end 112.635 77.565) (width 0.1524) (layer "B.Cu") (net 8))
 (segment (start 114 62.9793) (end 114.1293 62.85) (width 0.1524) (layer "F.Cu") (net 11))
 (segment (start 114.1293 62.85) (end 115.5 62.85) (width 0.1524) (layer "F.Cu") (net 11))
 (via (at 114 62.9793) (size 0.5842) (drill 0.3048) (layers "F.Cu" "B.Cu") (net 11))
 (segment (start 114 62.9793) (end 114.75 63.7293) (width 0.1524) (layer "B.Cu") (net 11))
 (segment (start 114.75 72.91) (end 112.635 75.025) (width 0.1524) (layer "B.Cu") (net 11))
 (segment (start 114.75 63.7293) (end 114.75 72.91) (width 0.1524) (layer "B.Cu") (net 11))
 (segment (start 116.349999 57.77) (end 115.5 57.77) (width 0.1524) (layer "F.Cu") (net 7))
 (segment (start 127.875 80.105) (end 118.5 70.73) (width 0.1524) (layer "F.Cu") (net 7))
 (segment (start 118.5 59.920001) (end 116.349999 57.77) (width 0.1524) (layer "F.Cu") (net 7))
 (segment (start 118.5 70.73) (end 118.5 59.920001) (width 0.1524) (layer "F.Cu") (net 7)))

